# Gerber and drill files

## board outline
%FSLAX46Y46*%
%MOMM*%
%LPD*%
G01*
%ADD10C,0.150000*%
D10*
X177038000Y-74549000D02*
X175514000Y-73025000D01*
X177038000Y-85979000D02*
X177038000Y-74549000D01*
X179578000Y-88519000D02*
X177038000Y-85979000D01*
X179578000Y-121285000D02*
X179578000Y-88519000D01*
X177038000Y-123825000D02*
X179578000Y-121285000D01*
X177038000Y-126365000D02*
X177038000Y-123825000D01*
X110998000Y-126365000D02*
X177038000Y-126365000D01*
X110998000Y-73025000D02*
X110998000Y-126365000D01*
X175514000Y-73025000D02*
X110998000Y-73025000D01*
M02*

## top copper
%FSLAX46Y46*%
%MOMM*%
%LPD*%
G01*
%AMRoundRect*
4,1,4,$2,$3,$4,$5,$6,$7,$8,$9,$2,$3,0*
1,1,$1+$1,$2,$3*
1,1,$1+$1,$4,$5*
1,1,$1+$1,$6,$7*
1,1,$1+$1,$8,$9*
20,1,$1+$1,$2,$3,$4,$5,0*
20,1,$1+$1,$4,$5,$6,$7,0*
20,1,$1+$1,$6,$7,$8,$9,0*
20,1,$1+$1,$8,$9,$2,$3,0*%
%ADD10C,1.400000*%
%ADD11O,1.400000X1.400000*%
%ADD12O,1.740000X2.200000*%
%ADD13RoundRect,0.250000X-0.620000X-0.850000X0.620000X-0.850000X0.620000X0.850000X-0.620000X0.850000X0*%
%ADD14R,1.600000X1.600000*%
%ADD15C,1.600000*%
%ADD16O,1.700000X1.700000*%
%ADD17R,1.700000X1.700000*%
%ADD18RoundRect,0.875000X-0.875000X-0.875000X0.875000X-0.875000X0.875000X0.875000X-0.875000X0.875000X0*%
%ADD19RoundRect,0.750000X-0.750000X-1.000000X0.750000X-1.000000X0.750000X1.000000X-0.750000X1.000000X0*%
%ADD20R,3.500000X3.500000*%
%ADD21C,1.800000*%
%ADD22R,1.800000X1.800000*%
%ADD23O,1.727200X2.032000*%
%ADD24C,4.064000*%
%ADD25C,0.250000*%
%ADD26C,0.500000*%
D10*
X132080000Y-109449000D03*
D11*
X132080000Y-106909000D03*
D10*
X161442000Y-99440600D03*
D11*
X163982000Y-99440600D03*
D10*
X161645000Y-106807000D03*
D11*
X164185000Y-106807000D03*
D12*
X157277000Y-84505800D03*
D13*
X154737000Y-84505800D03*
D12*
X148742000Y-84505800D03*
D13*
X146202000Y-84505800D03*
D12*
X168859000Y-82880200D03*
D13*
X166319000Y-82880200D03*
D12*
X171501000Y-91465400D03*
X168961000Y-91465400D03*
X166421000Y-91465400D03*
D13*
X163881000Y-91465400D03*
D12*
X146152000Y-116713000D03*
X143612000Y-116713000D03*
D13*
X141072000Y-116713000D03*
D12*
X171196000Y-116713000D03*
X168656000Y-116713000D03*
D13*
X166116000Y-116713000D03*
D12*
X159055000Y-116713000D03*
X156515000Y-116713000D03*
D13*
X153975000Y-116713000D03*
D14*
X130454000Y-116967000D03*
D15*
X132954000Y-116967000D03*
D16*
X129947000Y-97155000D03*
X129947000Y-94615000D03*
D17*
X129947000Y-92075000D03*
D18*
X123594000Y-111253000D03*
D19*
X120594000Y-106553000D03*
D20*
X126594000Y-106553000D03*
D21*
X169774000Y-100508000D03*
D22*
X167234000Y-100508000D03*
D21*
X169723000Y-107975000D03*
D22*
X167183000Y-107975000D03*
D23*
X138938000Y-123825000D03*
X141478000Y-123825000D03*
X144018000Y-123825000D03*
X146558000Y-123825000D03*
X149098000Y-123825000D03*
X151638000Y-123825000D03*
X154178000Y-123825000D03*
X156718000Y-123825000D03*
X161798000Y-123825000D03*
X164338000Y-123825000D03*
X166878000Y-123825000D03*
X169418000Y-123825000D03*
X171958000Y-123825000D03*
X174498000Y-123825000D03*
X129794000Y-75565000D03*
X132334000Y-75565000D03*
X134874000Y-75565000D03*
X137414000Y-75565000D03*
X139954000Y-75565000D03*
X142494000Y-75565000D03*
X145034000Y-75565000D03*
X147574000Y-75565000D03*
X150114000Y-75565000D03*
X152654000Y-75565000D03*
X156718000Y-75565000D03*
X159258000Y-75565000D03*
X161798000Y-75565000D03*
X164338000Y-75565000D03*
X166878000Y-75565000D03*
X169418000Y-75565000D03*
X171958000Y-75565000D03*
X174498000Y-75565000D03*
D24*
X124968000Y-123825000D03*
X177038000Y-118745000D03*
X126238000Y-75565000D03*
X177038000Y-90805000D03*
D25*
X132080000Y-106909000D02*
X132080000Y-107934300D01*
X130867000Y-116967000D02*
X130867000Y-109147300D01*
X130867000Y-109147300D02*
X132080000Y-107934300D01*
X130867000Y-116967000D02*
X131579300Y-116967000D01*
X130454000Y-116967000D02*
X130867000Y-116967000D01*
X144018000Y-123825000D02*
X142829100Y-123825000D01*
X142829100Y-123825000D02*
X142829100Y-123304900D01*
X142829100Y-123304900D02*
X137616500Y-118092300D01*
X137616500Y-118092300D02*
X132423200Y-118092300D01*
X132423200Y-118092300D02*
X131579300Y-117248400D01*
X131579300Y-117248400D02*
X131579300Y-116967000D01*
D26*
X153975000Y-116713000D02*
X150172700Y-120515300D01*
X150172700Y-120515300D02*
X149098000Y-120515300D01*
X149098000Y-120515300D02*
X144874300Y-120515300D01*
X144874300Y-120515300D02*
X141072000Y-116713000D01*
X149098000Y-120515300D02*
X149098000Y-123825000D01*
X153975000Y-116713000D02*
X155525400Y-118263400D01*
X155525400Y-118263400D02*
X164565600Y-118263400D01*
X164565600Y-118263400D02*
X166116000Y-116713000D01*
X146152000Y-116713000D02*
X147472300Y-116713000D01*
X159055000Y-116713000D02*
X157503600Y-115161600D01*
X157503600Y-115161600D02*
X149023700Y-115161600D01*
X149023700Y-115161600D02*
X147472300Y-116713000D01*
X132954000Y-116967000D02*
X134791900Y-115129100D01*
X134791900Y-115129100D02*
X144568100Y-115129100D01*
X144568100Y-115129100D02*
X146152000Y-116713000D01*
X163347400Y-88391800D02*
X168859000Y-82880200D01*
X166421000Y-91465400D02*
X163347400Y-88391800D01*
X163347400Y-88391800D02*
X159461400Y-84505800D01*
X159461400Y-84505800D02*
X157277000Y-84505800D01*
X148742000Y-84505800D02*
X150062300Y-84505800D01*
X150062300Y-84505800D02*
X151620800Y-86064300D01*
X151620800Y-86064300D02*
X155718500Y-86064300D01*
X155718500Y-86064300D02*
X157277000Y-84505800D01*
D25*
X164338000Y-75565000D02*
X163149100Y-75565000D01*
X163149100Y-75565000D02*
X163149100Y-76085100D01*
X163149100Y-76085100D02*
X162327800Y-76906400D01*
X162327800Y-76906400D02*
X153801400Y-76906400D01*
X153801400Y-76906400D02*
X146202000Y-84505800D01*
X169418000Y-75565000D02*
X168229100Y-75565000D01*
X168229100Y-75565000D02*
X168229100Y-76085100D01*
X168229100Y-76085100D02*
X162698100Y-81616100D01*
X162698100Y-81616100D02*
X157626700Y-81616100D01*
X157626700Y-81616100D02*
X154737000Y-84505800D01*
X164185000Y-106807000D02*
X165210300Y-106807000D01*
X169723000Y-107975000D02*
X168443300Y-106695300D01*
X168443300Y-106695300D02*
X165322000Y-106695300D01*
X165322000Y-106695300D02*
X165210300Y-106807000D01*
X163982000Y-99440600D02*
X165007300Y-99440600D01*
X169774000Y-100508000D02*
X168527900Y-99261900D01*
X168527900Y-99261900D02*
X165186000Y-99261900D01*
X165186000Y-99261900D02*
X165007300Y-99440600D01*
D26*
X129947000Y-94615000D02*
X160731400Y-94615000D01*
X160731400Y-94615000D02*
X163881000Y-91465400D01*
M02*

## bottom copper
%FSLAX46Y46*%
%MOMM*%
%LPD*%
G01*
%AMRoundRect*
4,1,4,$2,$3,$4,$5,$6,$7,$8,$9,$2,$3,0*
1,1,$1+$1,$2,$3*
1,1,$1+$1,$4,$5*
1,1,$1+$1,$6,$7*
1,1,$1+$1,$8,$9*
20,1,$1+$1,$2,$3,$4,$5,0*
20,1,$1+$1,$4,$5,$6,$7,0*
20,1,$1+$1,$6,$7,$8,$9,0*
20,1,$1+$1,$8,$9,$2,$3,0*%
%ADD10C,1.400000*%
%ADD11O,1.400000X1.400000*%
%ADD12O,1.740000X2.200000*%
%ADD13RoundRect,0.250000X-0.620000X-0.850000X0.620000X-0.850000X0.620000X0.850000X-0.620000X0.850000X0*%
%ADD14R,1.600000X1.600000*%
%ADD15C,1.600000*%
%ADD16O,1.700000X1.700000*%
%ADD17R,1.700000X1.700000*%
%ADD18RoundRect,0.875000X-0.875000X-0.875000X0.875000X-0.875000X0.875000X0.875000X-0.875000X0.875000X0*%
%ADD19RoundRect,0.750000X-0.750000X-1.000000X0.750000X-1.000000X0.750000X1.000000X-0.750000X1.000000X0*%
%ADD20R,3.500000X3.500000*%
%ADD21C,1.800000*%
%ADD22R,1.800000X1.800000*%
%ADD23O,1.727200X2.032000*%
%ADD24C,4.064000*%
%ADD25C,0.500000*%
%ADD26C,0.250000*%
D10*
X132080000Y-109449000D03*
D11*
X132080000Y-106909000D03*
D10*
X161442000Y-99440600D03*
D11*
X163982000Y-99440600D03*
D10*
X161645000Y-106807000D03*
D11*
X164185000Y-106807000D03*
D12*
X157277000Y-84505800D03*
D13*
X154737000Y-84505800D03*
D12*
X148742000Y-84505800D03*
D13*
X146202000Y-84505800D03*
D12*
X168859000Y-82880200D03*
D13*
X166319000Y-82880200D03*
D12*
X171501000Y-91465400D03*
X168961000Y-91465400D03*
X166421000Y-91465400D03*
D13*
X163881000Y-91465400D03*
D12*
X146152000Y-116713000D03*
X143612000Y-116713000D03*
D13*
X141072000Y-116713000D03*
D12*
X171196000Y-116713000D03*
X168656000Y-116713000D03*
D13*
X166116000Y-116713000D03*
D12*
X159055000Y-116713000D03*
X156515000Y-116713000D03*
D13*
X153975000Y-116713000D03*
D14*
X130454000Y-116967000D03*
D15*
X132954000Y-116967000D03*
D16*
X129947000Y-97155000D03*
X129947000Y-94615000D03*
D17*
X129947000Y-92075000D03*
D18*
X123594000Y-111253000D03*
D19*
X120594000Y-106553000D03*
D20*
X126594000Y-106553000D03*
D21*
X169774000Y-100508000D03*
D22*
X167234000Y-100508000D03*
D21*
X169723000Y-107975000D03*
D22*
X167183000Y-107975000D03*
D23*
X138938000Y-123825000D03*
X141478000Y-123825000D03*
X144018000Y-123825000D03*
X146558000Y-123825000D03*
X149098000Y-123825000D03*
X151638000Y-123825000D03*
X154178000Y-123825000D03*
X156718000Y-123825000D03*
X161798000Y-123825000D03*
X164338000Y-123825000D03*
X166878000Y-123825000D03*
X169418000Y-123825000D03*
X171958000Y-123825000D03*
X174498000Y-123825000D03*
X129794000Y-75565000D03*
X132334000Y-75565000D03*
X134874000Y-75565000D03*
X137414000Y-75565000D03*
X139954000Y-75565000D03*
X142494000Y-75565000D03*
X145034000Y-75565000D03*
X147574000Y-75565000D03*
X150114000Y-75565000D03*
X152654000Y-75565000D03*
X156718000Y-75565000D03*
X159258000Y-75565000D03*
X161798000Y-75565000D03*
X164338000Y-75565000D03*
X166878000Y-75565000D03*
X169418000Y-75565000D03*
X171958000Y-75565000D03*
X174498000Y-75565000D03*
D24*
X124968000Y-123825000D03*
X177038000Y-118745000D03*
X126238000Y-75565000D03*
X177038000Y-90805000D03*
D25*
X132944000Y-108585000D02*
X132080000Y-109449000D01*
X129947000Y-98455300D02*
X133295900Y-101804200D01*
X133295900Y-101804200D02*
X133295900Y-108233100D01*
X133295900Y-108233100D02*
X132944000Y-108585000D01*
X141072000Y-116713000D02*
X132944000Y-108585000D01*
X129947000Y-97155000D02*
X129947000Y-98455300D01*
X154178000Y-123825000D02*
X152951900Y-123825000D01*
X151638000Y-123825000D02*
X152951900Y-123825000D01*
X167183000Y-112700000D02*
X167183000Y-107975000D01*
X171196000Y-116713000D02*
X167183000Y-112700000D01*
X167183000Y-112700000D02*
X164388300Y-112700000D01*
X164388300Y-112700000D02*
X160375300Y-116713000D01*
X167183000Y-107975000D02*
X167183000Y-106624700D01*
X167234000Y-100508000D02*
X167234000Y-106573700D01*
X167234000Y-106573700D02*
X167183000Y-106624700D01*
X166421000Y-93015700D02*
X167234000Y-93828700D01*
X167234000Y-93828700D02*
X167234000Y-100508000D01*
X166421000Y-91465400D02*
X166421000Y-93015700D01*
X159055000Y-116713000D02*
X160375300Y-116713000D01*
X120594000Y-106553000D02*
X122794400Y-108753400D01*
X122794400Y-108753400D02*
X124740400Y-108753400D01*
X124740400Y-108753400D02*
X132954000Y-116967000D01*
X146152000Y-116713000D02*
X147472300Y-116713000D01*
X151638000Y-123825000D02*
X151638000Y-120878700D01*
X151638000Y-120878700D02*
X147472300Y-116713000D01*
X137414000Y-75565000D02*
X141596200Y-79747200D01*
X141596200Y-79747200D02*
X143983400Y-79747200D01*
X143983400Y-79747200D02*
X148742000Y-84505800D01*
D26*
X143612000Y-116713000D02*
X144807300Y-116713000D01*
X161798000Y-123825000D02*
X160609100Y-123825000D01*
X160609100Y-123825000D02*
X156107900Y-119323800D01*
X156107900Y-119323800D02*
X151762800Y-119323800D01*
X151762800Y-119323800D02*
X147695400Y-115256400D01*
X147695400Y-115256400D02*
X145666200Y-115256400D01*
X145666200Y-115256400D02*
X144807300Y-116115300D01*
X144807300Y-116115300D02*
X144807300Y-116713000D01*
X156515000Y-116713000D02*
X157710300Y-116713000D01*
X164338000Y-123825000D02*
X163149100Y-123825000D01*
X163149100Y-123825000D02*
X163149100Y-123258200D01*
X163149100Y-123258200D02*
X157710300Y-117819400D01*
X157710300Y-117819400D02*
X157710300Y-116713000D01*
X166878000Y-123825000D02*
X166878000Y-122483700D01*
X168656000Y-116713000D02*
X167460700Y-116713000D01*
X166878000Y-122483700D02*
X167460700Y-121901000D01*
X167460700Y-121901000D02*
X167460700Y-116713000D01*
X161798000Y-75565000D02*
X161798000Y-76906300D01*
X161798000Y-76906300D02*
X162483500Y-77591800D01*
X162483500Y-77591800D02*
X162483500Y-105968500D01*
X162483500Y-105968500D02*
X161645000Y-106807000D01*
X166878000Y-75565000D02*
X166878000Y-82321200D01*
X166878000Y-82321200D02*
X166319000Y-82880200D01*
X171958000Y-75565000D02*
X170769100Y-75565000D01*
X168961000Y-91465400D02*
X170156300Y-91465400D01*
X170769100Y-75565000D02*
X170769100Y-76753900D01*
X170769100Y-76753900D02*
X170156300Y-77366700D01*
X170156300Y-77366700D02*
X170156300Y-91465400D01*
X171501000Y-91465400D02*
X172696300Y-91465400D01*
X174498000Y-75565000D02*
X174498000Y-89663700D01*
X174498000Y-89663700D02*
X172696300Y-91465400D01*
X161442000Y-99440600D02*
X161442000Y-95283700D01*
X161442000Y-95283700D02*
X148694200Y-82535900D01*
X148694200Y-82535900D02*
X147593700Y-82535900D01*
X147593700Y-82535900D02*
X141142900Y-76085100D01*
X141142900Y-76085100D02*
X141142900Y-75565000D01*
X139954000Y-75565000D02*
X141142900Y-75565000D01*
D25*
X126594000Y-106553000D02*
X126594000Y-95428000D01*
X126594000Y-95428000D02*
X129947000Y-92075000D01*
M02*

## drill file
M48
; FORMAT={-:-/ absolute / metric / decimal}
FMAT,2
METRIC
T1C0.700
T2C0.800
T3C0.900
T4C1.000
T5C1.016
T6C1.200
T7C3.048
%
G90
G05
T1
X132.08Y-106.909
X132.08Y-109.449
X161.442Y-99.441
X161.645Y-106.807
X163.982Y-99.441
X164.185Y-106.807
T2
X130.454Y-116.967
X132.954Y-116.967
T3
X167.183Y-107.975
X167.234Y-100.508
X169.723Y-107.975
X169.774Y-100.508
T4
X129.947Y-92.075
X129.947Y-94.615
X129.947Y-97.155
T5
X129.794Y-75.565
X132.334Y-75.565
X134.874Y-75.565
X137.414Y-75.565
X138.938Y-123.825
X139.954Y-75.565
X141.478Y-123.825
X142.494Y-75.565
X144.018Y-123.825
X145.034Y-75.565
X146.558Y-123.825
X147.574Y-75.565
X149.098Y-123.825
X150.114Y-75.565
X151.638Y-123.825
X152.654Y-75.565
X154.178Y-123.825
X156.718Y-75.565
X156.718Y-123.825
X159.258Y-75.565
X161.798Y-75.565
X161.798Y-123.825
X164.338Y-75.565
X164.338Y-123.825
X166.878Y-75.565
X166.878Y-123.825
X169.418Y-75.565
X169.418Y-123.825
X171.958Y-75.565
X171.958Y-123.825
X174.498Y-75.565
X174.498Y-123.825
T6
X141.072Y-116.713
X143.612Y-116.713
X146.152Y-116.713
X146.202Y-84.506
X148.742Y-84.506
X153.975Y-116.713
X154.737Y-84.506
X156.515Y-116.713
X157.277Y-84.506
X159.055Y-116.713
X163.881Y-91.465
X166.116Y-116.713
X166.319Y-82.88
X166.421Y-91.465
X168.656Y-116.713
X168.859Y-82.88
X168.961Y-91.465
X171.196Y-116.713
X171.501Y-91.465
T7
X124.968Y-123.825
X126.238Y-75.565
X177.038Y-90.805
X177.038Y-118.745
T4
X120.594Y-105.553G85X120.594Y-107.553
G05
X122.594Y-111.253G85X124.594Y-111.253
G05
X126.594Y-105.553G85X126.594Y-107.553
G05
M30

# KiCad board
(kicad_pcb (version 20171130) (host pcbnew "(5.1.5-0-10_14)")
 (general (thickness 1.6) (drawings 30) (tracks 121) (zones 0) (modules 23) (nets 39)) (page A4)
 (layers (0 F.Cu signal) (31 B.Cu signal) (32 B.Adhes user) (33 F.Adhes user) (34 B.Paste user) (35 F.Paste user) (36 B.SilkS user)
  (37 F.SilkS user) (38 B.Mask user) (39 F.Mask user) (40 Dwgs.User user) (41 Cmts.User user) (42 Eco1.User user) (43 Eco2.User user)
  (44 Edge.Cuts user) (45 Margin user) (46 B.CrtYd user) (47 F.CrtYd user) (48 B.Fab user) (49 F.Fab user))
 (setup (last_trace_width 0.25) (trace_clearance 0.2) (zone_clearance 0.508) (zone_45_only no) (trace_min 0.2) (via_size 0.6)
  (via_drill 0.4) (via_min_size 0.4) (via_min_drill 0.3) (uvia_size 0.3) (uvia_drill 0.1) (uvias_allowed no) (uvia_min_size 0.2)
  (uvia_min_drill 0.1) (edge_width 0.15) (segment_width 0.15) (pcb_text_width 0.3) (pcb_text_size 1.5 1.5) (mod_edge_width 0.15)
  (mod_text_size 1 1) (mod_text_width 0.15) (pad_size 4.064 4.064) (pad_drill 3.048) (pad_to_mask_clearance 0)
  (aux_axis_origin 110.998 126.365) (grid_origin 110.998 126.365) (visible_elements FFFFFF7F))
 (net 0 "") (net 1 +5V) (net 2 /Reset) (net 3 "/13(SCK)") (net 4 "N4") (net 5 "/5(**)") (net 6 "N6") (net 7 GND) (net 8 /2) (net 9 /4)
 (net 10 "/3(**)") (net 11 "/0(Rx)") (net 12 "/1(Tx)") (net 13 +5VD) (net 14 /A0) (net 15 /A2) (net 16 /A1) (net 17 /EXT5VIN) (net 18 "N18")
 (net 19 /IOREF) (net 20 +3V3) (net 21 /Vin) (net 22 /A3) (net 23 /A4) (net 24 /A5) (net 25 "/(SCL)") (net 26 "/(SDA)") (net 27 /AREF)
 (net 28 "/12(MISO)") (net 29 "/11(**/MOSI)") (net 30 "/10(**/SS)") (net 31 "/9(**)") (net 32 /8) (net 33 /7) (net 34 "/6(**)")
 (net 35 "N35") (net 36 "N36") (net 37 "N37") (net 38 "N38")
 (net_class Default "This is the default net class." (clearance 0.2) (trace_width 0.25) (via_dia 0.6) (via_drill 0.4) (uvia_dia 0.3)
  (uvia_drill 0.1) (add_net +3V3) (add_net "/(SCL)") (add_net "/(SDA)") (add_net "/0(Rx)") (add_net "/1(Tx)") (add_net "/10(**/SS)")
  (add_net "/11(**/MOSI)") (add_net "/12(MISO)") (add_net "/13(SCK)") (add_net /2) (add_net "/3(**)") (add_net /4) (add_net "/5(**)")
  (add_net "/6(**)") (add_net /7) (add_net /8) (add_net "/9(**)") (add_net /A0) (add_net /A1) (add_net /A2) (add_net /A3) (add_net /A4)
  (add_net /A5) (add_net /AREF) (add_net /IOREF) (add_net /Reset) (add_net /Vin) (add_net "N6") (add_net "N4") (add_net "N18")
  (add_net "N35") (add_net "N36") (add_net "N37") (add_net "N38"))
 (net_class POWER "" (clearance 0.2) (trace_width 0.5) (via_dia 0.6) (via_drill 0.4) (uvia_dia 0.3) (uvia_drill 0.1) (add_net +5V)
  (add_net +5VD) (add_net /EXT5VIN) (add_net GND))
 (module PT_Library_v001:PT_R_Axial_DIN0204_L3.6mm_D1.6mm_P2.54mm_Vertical (layer F.Cu) (at 132.08 109.449 90)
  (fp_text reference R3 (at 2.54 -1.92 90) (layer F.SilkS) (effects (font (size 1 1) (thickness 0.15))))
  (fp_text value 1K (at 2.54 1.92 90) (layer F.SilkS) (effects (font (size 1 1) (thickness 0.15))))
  (pad 1 thru_hole circle (at 0 0 90) (size 1.4 1.4) (drill 0.7) (layers *.Cu *.Mask) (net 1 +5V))
  (pad 2 thru_hole oval (at 2.54 0 90) (size 1.4 1.4) (drill 0.7) (layers *.Cu *.Mask) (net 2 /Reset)))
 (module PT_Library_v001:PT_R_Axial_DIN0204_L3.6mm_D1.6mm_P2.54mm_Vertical (layer F.Cu) (at 161.442 99.4406)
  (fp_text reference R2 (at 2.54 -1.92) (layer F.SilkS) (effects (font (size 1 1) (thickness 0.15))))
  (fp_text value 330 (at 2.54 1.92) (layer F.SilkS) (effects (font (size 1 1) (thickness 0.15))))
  (pad 1 thru_hole circle (at 0 0) (size 1.4 1.4) (drill 0.7) (layers *.Cu *.Mask) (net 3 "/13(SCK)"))
  (pad 2 thru_hole oval (at 2.54 0) (size 1.4 1.4) (drill 0.7) (layers *.Cu *.Mask) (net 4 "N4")))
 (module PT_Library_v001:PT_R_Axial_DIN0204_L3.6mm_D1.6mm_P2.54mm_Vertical (layer F.Cu) (at 161.645 106.807)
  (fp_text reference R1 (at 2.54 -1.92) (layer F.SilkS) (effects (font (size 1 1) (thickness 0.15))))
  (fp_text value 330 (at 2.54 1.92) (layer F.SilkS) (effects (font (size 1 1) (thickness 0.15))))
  (pad 1 thru_hole circle (at 0 0) (size 1.4 1.4) (drill 0.7) (layers *.Cu *.Mask) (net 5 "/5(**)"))
  (pad 2 thru_hole oval (at 2.54 0) (size 1.4 1.4) (drill 0.7) (layers *.Cu *.Mask) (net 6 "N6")))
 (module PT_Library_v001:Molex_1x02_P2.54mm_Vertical (layer F.Cu) (at 154.737 84.5058)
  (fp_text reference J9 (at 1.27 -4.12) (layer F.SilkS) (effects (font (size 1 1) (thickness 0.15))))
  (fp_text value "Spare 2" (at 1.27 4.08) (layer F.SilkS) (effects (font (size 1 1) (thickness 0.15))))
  (pad 2 thru_hole oval (at 2.54 0) (size 1.74 2.2) (drill 1.2) (layers *.Cu *.Mask) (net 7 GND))
  (pad 1 thru_hole roundrect (at 0 0) (size 1.74 2.2) (drill 1.2) (layers *.Cu *.Mask) (roundrect_rratio 0.143678) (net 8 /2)))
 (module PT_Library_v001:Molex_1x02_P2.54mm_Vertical (layer F.Cu) (at 146.202 84.5058)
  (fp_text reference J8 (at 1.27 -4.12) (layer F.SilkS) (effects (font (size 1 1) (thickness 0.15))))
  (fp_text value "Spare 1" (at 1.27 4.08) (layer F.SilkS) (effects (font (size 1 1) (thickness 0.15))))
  (pad 2 thru_hole oval (at 2.54 0) (size 1.74 2.2) (drill 1.2) (layers *.Cu *.Mask) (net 7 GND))
  (pad 1 thru_hole roundrect (at 0 0) (size 1.74 2.2) (drill 1.2) (layers *.Cu *.Mask) (roundrect_rratio 0.143678) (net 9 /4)))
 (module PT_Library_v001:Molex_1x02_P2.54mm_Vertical (layer F.Cu) (at 166.319 82.8802)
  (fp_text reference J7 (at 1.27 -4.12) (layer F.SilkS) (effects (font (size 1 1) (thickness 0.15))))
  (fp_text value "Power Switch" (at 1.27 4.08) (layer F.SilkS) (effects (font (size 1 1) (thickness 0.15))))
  (pad 2 thru_hole oval (at 2.54 0) (size 1.74 2.2) (drill 1.2) (layers *.Cu *.Mask) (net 7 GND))
  (pad 1 thru_hole roundrect (at 0 0) (size 1.74 2.2) (drill 1.2) (layers *.Cu *.Mask) (roundrect_rratio 0.143678) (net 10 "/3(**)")))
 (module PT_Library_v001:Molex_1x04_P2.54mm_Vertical (layer F.Cu) (at 163.881 91.4654)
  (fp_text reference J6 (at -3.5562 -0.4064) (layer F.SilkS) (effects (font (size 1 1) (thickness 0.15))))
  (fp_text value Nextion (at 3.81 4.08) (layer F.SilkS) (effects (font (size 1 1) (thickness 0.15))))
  (pad 4 thru_hole oval (at 7.62 0) (size 1.74 2.2) (drill 1.2) (layers *.Cu *.Mask) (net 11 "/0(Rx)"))
  (pad 3 thru_hole oval (at 5.08 0) (size 1.74 2.2) (drill 1.2) (layers *.Cu *.Mask) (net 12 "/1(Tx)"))
  (pad 2 thru_hole oval (at 2.54 0) (size 1.74 2.2) (drill 1.2) (layers *.Cu *.Mask) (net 7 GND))
  (pad 1 thru_hole roundrect (at 0 0) (size 1.74 2.2) (drill 1.2) (layers *.Cu *.Mask) (roundrect_rratio 0.143678) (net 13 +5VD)))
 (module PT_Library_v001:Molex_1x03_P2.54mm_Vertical (layer F.Cu) (at 141.072 116.713)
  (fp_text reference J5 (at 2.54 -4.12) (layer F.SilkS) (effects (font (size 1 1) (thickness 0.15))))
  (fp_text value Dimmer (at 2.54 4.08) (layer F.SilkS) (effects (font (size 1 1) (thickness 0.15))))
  (pad 3 thru_hole oval (at 5.08 0) (size 1.74 2.2) (drill 1.2) (layers *.Cu *.Mask) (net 7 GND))
  (pad 2 thru_hole oval (at 2.54 0) (size 1.74 2.2) (drill 1.2) (layers *.Cu *.Mask) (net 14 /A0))
  (pad 1 thru_hole roundrect (at 0 0) (size 1.74 2.2) (drill 1.2) (layers *.Cu *.Mask) (roundrect_rratio 0.143678) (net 1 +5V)))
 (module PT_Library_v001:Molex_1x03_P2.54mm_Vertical (layer F.Cu) (at 166.116 116.713)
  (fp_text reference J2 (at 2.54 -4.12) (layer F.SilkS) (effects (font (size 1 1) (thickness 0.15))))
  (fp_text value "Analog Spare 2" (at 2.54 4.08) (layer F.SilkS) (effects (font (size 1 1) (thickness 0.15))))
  (pad 3 thru_hole oval (at 5.08 0) (size 1.74 2.2) (drill 1.2) (layers *.Cu *.Mask) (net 7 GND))
  (pad 2 thru_hole oval (at 2.54 0) (size 1.74 2.2) (drill 1.2) (layers *.Cu *.Mask) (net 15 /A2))
  (pad 1 thru_hole roundrect (at 0 0) (size 1.74 2.2) (drill 1.2) (layers *.Cu *.Mask) (roundrect_rratio 0.143678) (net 1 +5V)))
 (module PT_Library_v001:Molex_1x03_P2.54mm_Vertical (layer F.Cu) (at 153.975 116.713)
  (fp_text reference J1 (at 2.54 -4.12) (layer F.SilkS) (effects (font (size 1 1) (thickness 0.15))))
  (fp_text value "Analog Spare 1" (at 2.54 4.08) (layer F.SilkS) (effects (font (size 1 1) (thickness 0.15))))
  (pad 3 thru_hole oval (at 5.08 0) (size 1.74 2.2) (drill 1.2) (layers *.Cu *.Mask) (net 7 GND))
  (pad 2 thru_hole oval (at 2.54 0) (size 1.74 2.2) (drill 1.2) (layers *.Cu *.Mask) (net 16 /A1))
  (pad 1 thru_hole roundrect (at 0 0) (size 1.74 2.2) (drill 1.2) (layers *.Cu *.Mask) (roundrect_rratio 0.143678) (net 1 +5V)))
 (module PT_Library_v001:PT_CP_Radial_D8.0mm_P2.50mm (layer F.Cu) (at 130.454 116.967)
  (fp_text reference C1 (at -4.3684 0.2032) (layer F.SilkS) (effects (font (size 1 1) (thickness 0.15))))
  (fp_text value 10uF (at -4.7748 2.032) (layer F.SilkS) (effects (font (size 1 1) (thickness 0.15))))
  (pad 1 thru_hole rect (at 0 0) (size 1.6 1.6) (drill 0.8) (layers *.Cu *.Mask) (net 2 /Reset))
  (pad 2 thru_hole circle (at 2.5 0) (size 1.6 1.6) (drill 0.8) (layers *.Cu *.Mask) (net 7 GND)))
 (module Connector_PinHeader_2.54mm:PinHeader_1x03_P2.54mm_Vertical (layer F.Cu) (at 129.947 92.075)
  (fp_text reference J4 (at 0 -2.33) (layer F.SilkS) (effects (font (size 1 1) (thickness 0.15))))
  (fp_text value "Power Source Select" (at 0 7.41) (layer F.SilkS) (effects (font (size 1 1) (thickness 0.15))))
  (pad 3 thru_hole oval (at 0 5.08) (size 1.7 1.7) (drill 1) (layers *.Cu *.Mask) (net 1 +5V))
  (pad 2 thru_hole oval (at 0 2.54) (size 1.7 1.7) (drill 1) (layers *.Cu *.Mask) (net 13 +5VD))
  (pad 1 thru_hole rect (at 0 0) (size 1.7 1.7) (drill 1) (layers *.Cu *.Mask) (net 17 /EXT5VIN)))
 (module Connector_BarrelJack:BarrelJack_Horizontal (layer F.Cu) (at 126.594 106.553)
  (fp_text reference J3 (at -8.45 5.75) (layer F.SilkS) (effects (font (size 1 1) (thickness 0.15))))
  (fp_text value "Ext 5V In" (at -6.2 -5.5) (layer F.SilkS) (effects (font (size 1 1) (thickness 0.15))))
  (pad 3 thru_hole roundrect (at -3 4.7) (size 3.5 3.5) (drill oval 3 1) (layers *.Cu *.Mask) (roundrect_rratio 0.25))
  (pad 2 thru_hole roundrect (at -6 0) (size 3 3.5) (drill oval 1 3) (layers *.Cu *.Mask) (roundrect_rratio 0.25) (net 7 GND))
  (pad 1 thru_hole rect (at 0 0) (size 3.5 3.5) (drill oval 1 3) (layers *.Cu *.Mask) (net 17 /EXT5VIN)))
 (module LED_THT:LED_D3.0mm (layer F.Cu) (at 167.234 100.508)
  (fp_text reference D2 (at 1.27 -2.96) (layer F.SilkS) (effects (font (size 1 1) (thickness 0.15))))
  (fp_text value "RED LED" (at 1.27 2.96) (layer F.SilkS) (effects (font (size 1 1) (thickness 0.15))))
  (pad 2 thru_hole circle (at 2.54 0) (size 1.8 1.8) (drill 0.9) (layers *.Cu *.Mask) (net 4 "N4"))
  (pad 1 thru_hole rect (at 0 0) (size 1.8 1.8) (drill 0.9) (layers *.Cu *.Mask) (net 7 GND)))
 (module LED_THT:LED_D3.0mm (layer F.Cu) (at 167.183 107.975)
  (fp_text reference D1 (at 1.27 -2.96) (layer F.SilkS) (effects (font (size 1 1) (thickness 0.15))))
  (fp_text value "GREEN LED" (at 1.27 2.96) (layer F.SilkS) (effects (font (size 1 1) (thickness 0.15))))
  (pad 2 thru_hole circle (at 2.54 0) (size 1.8 1.8) (drill 0.9) (layers *.Cu *.Mask) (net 6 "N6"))
  (pad 1 thru_hole rect (at 0 0) (size 1.8 1.8) (drill 0.9) (layers *.Cu *.Mask) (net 7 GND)))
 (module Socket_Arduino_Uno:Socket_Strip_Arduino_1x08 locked (layer F.Cu) (at 138.938 123.825)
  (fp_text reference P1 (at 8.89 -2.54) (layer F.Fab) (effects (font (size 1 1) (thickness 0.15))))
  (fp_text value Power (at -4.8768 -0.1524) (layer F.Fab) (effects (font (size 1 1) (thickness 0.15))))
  (pad 1 thru_hole oval (at 0 0) (size 1.7272 2.032) (drill 1.016) (layers *.Cu *.Mask F.SilkS) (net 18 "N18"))
  (pad 2 thru_hole oval (at 2.54 0) (size 1.7272 2.032) (drill 1.016) (layers *.Cu *.Mask F.SilkS) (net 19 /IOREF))
  (pad 3 thru_hole oval (at 5.08 0) (size 1.7272 2.032) (drill 1.016) (layers *.Cu *.Mask F.SilkS) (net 2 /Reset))
  (pad 4 thru_hole oval (at 7.62 0) (size 1.7272 2.032) (drill 1.016) (layers *.Cu *.Mask F.SilkS) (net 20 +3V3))
  (pad 5 thru_hole oval (at 10.16 0) (size 1.7272 2.032) (drill 1.016) (layers *.Cu *.Mask F.SilkS) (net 1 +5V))
  (pad 6 thru_hole oval (at 12.7 0) (size 1.7272 2.032) (drill 1.016) (layers *.Cu *.Mask F.SilkS) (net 7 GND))
  (pad 7 thru_hole oval (at 15.24 0) (size 1.7272 2.032) (drill 1.016) (layers *.Cu *.Mask F.SilkS) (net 7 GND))
  (pad 8 thru_hole oval (at 17.78 0) (size 1.7272 2.032) (drill 1.016) (layers *.Cu *.Mask F.SilkS) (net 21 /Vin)))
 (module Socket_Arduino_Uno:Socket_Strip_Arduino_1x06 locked (layer F.Cu) (at 161.798 123.825)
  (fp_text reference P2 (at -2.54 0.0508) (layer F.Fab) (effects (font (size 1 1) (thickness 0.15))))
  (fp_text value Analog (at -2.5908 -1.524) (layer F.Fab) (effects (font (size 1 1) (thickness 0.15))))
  (pad 1 thru_hole oval (at 0 0) (size 1.7272 2.032) (drill 1.016) (layers *.Cu *.Mask F.SilkS) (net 14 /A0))
  (pad 2 thru_hole oval (at 2.54 0) (size 1.7272 2.032) (drill 1.016) (layers *.Cu *.Mask F.SilkS) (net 16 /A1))
  (pad 3 thru_hole oval (at 5.08 0) (size 1.7272 2.032) (drill 1.016) (layers *.Cu *.Mask F.SilkS) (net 15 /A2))
  (pad 4 thru_hole oval (at 7.62 0) (size 1.7272 2.032) (drill 1.016) (layers *.Cu *.Mask F.SilkS) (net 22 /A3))
  (pad 5 thru_hole oval (at 10.16 0) (size 1.7272 2.032) (drill 1.016) (layers *.Cu *.Mask F.SilkS) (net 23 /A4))
  (pad 6 thru_hole oval (at 12.7 0) (size 1.7272 2.032) (drill 1.016) (layers *.Cu *.Mask F.SilkS) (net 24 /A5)))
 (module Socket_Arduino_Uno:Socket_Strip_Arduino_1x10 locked (layer F.Cu) (at 129.794 75.565)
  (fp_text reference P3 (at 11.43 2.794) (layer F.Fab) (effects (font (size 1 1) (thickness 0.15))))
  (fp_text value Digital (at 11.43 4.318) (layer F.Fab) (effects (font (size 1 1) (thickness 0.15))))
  (pad 1 thru_hole oval (at 0 0) (size 1.7272 2.032) (drill 1.016) (layers *.Cu *.Mask F.SilkS) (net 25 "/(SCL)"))
  (pad 2 thru_hole oval (at 2.54 0) (size 1.7272 2.032) (drill 1.016) (layers *.Cu *.Mask F.SilkS) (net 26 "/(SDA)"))
  (pad 3 thru_hole oval (at 5.08 0) (size 1.7272 2.032) (drill 1.016) (layers *.Cu *.Mask F.SilkS) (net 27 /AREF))
  (pad 4 thru_hole oval (at 7.62 0) (size 1.7272 2.032) (drill 1.016) (layers *.Cu *.Mask F.SilkS) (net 7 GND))
  (pad 5 thru_hole oval (at 10.16 0) (size 1.7272 2.032) (drill 1.016) (layers *.Cu *.Mask F.SilkS) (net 3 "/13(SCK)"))
  (pad 6 thru_hole oval (at 12.7 0) (size 1.7272 2.032) (drill 1.016) (layers *.Cu *.Mask F.SilkS) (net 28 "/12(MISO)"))
  (pad 7 thru_hole oval (at 15.24 0) (size 1.7272 2.032) (drill 1.016) (layers *.Cu *.Mask F.SilkS) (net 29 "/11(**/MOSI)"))
  (pad 8 thru_hole oval (at 17.78 0) (size 1.7272 2.032) (drill 1.016) (layers *.Cu *.Mask F.SilkS) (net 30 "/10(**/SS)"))
  (pad 9 thru_hole oval (at 20.32 0) (size 1.7272 2.032) (drill 1.016) (layers *.Cu *.Mask F.SilkS) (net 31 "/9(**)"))
  (pad 10 thru_hole oval (at 22.86 0) (size 1.7272 2.032) (drill 1.016) (layers *.Cu *.Mask F.SilkS) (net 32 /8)))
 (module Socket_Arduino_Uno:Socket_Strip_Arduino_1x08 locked (layer F.Cu) (at 156.718 75.565)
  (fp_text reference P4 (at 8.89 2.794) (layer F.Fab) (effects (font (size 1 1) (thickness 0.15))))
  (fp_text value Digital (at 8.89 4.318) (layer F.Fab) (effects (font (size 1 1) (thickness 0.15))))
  (pad 1 thru_hole oval (at 0 0) (size 1.7272 2.032) (drill 1.016) (layers *.Cu *.Mask F.SilkS) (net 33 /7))
  (pad 2 thru_hole oval (at 2.54 0) (size 1.7272 2.032) (drill 1.016) (layers *.Cu *.Mask F.SilkS) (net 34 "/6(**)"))
  (pad 3 thru_hole oval (at 5.08 0) (size 1.7272 2.032) (drill 1.016) (layers *.Cu *.Mask F.SilkS) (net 5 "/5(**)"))
  (pad 4 thru_hole oval (at 7.62 0) (size 1.7272 2.032) (drill 1.016) (layers *.Cu *.Mask F.SilkS) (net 9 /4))
  (pad 5 thru_hole oval (at 10.16 0) (size 1.7272 2.032) (drill 1.016) (layers *.Cu *.Mask F.SilkS) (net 10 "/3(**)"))
  (pad 6 thru_hole oval (at 12.7 0) (size 1.7272 2.032) (drill 1.016) (layers *.Cu *.Mask F.SilkS) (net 8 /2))
  (pad 7 thru_hole oval (at 15.24 0) (size 1.7272 2.032) (drill 1.016) (layers *.Cu *.Mask F.SilkS) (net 12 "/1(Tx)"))
  (pad 8 thru_hole oval (at 17.78 0) (size 1.7272 2.032) (drill 1.016) (layers *.Cu *.Mask F.SilkS) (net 11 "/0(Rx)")))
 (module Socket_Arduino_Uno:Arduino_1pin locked (layer F.Cu) (at 124.968 123.825)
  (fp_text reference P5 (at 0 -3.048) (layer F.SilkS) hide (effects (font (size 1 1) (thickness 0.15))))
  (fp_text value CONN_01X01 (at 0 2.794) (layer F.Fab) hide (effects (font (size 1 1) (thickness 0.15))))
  (pad 1 thru_hole circle (at 0 0) (size 4.064 4.064) (drill 3.048) (layers *.Cu *.Mask F.SilkS) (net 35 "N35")))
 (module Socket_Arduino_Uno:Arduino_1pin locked (layer F.Cu) (at 177.038 118.745)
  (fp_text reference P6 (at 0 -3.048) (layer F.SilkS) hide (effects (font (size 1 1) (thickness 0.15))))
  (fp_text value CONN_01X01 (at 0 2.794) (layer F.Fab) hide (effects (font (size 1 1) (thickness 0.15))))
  (pad 1 thru_hole circle (at 0 0) (size 4.064 4.064) (drill 3.048) (layers *.Cu *.Mask F.SilkS) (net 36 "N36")))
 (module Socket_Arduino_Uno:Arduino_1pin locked (layer F.Cu) (at 126.238 75.565)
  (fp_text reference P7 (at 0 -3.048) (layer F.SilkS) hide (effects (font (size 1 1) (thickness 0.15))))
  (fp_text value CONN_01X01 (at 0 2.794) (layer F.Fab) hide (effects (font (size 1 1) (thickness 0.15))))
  (pad 1 thru_hole circle (at 0 0) (size 4.064 4.064) (drill 3.048) (layers *.Cu *.Mask F.SilkS) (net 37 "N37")))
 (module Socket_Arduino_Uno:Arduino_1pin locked (layer F.Cu) (at 177.038 90.805)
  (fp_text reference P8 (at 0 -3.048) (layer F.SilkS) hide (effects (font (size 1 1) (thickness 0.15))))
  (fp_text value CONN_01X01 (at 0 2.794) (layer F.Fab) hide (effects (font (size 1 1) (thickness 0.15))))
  (pad 1 thru_hole circle (at 0 0) (size 4.064 4.064) (drill 3.048) (layers *.Cu *.Mask F.SilkS) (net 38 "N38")))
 (gr_line (start 177.038 74.549) (end 175.514 73.025) (angle 90) (layer Edge.Cuts) (width 0.15))
 (gr_line (start 177.038 85.979) (end 177.038 74.549) (angle 90) (layer Edge.Cuts) (width 0.15))
 (gr_line (start 179.578 88.519) (end 177.038 85.979) (angle 90) (layer Edge.Cuts) (width 0.15))
 (gr_line (start 179.578 121.285) (end 179.578 88.519) (angle 90) (layer Edge.Cuts) (width 0.15))
 (gr_line (start 177.038 123.825) (end 179.578 121.285) (angle 90) (layer Edge.Cuts) (width 0.15))
 (gr_line (start 177.038 126.365) (end 177.038 123.825) (angle 90) (layer Edge.Cuts) (width 0.15))
 (gr_line (start 110.998 126.365) (end 177.038 126.365) (angle 90) (layer Edge.Cuts) (width 0.15))
 (gr_line (start 110.998 73.025) (end 110.998 126.365) (angle 90) (layer Edge.Cuts) (width 0.15))
 (gr_line (start 175.514 73.025) (end 110.998 73.025) (angle 90) (layer Edge.Cuts) (width 0.15))
 (segment (start 132.08 106.909) (end 132.08 107.9343) (width 0.25) (layer F.Cu) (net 2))
 (segment (start 130.867 116.967) (end 130.867 109.1473) (width 0.25) (layer F.Cu) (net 2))
 (segment (start 130.867 109.1473) (end 132.08 107.9343) (width 0.25) (layer F.Cu) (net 2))
 (segment (start 130.867 116.967) (end 131.5793 116.967) (width 0.25) (layer F.Cu) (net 2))
 (segment (start 130.454 116.967) (end 130.867 116.967) (width 0.25) (layer F.Cu) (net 2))
 (segment (start 144.018 123.825) (end 142.8291 123.825) (width 0.25) (layer F.Cu) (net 2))
 (segment (start 142.8291 123.825) (end 142.8291 123.3049) (width 0.25) (layer F.Cu) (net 2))
 (segment (start 142.8291 123.3049) (end 137.6165 118.0923) (width 0.25) (layer F.Cu) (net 2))
 (segment (start 137.6165 118.0923) (end 132.4232 118.0923) (width 0.25) (layer F.Cu) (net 2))
 (segment (start 132.4232 118.0923) (end 131.5793 117.2484) (width 0.25) (layer F.Cu) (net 2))
 (segment (start 131.5793 117.2484) (end 131.5793 116.967) (width 0.25) (layer F.Cu) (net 2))
 (segment (start 153.975 116.713) (end 150.1727 120.5153) (width 0.5) (layer F.Cu) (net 1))
 (segment (start 150.1727 120.5153) (end 149.098 120.5153) (width 0.5) (layer F.Cu) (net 1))
 (segment (start 149.098 120.5153) (end 144.8743 120.5153) (width 0.5) (layer F.Cu) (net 1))
 (segment (start 144.8743 120.5153) (end 141.072 116.713) (width 0.5) (layer F.Cu) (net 1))
 (segment (start 149.098 120.5153) (end 149.098 123.825) (width 0.5) (layer F.Cu) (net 1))
 (segment (start 153.975 116.713) (end 155.5254 118.2634) (width 0.5) (layer F.Cu) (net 1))
 (segment (start 155.5254 118.2634) (end 164.5656 118.2634) (width 0.5) (layer F.Cu) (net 1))
 (segment (start 164.5656 118.2634) (end 166.116 116.713) (width 0.5) (layer F.Cu) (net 1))
 (segment (start 132.944 108.585) (end 132.08 109.449) (width 0.5) (layer B.Cu) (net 1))
 (segment (start 129.947 98.4553) (end 133.2959 101.8042) (width 0.5) (layer B.Cu) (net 1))
 (segment (start 133.2959 101.8042) (end 133.2959 108.2331) (width 0.5) (layer B.Cu) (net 1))
 (segment (start 133.2959 108.2331) (end 132.944 108.585) (width 0.5) (layer B.Cu) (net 1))
 (segment (start 141.072 116.713) (end 132.944 108.585) (width 0.5) (layer B.Cu) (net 1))
 (segment (start 129.947 97.155) (end 129.947 98.4553) (width 0.5) (layer B.Cu) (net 1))
 (segment (start 146.152 116.713) (end 147.4723 116.713) (width 0.5) (layer F.Cu) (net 7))
 (segment (start 159.055 116.713) (end 157.5036 115.1616) (width 0.5) (layer F.Cu) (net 7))
 (segment (start 157.5036 115.1616) (end 149.0237 115.1616) (width 0.5) (layer F.Cu) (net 7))
 (segment (start 149.0237 115.1616) (end 147.4723 116.713) (width 0.5) (layer F.Cu) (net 7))
 (segment (start 132.954 116.967) (end 134.7919 115.1291) (width 0.5) (layer F.Cu) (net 7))
 (segment (start 134.7919 115.1291) (end 144.5681 115.1291) (width 0.5) (layer F.Cu) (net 7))
 (segment (start 144.5681 115.1291) (end 146.152 116.713) (width 0.5) (layer F.Cu) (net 7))
 (segment (start 163.3474 88.3918) (end 168.859 82.8802) (width 0.5) (layer F.Cu) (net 7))
 (segment (start 166.421 91.4654) (end 163.3474 88.3918) (width 0.5) (layer F.Cu) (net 7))
 (segment (start 163.3474 88.3918) (end 159.4614 84.5058) (width 0.5) (layer F.Cu) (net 7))
 (segment (start 159.4614 84.5058) (end 157.277 84.5058) (width 0.5) (layer F.Cu) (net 7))
 (segment (start 148.742 84.5058) (end 150.0623 84.5058) (width 0.5) (layer F.Cu) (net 7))
 (segment (start 150.0623 84.5058) (end 151.6208 86.0643) (width 0.5) (layer F.Cu) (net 7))
 (segment (start 151.6208 86.0643) (end 155.7185 86.0643) (width 0.5) (layer F.Cu) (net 7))
 (segment (start 155.7185 86.0643) (end 157.277 84.5058) (width 0.5) (layer F.Cu) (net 7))
 (segment (start 154.178 123.825) (end 152.9519 123.825) (width 0.5) (layer B.Cu) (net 7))
 (segment (start 151.638 123.825) (end 152.9519 123.825) (width 0.5) (layer B.Cu) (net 7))
 (segment (start 167.183 112.7) (end 167.183 107.975) (width 0.5) (layer B.Cu) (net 7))
 (segment (start 171.196 116.713) (end 167.183 112.7) (width 0.5) (layer B.Cu) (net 7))
 (segment (start 167.183 112.7) (end 164.3883 112.7) (width 0.5) (layer B.Cu) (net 7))
 (segment (start 164.3883 112.7) (end 160.3753 116.713) (width 0.5) (layer B.Cu) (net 7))
 (segment (start 167.183 107.975) (end 167.183 106.6247) (width 0.5) (layer B.Cu) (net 7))
 (segment (start 167.234 100.508) (end 167.234 106.5737) (width 0.5) (layer B.Cu) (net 7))
 (segment (start 167.234 106.5737) (end 167.183 106.6247) (width 0.5) (layer B.Cu) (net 7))
 (segment (start 166.421 93.0157) (end 167.234 93.8287) (width 0.5) (layer B.Cu) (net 7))
 (segment (start 167.234 93.8287) (end 167.234 100.508) (width 0.5) (layer B.Cu) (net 7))
 (segment (start 166.421 91.4654) (end 166.421 93.0157) (width 0.5) (layer B.Cu) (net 7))
 (segment (start 159.055 116.713) (end 160.3753 116.713) (width 0.5) (layer B.Cu) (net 7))
 (segment (start 120.594 106.553) (end 122.7944 108.7534) (width 0.5) (layer B.Cu) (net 7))
 (segment (start 122.7944 108.7534) (end 124.7404 108.7534) (width 0.5) (layer B.Cu) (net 7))
 (segment (start 124.7404 108.7534) (end 132.954 116.967) (width 0.5) (layer B.Cu) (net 7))
 (segment (start 146.152 116.713) (end 147.4723 116.713) (width 0.5) (layer B.Cu) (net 7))
 (segment (start 151.638 123.825) (end 151.638 120.8787) (width 0.5) (layer B.Cu) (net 7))
 (segment (start 151.638 120.8787) (end 147.4723 116.713) (width 0.5) (layer B.Cu) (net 7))
 (segment (start 137.414 75.565) (end 141.5962 79.7472) (width 0.5) (layer B.Cu) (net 7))
 (segment (start 141.5962 79.7472) (end 143.9834 79.7472) (width 0.5) (layer B.Cu) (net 7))
 (segment (start 143.9834 79.7472) (end 148.742 84.5058) (width 0.5) (layer B.Cu) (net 7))
 (segment (start 143.612 116.713) (end 144.8073 116.713) (width 0.25) (layer B.Cu) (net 14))
 (segment (start 161.798 123.825) (end 160.6091 123.825) (width 0.25) (layer B.Cu) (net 14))
 (segment (start 160.6091 123.825) (end 156.1079 119.3238) (width 0.25) (layer B.Cu) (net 14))
 (segment (start 156.1079 119.3238) (end 151.7628 119.3238) (width 0.25) (layer B.Cu) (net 14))
 (segment (start 151.7628 119.3238) (end 147.6954 115.2564) (width 0.25) (layer B.Cu) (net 14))
 (segment (start 147.6954 115.2564) (end 145.6662 115.2564) (width 0.25) (layer B.Cu) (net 14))
 (segment (start 145.6662 115.2564) (end 144.8073 116.1153) (width 0.25) (layer B.Cu) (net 14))
 (segment (start 144.8073 116.1153) (end 144.8073 116.713) (width 0.25) (layer B.Cu) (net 14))
 (segment (start 156.515 116.713) (end 157.7103 116.713) (width 0.25) (layer B.Cu) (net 16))
 (segment (start 164.338 123.825) (end 163.1491 123.825) (width 0.25) (layer B.Cu) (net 16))
 (segment (start 163.1491 123.825) (end 163.1491 123.2582) (width 0.25) (layer B.Cu) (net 16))
 (segment (start 163.1491 123.2582) (end 157.7103 117.8194) (width 0.25) (layer B.Cu) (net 16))
 (segment (start 157.7103 117.8194) (end 157.7103 116.713) (width 0.25) (layer B.Cu) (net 16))
 (segment (start 166.878 123.825) (end 166.878 122.4837) (width 0.25) (layer B.Cu) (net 15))
 (segment (start 168.656 116.713) (end 167.4607 116.713) (width 0.25) (layer B.Cu) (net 15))
 (segment (start 166.878 122.4837) (end 167.4607 121.901) (width 0.25) (layer B.Cu) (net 15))
 (segment (start 167.4607 121.901) (end 167.4607 116.713) (width 0.25) (layer B.Cu) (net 15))
 (segment (start 161.798 75.565) (end 161.798 76.9063) (width 0.25) (layer B.Cu) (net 5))
 (segment (start 161.798 76.9063) (end 162.4835 77.5918) (width 0.25) (layer B.Cu) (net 5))
 (segment (start 162.4835 77.5918) (end 162.4835 105.9685) (width 0.25) (layer B.Cu) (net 5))
 (segment (start 162.4835 105.9685) (end 161.645 106.807) (width 0.25) (layer B.Cu) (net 5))
 (segment (start 164.338 75.565) (end 163.1491 75.565) (width 0.25) (layer F.Cu) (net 9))
 (segment (start 163.1491 75.565) (end 163.1491 76.0851) (width 0.25) (layer F.Cu) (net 9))
 (segment (start 163.1491 76.0851) (end 162.3278 76.9064) (width 0.25) (layer F.Cu) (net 9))
 (segment (start 162.3278 76.9064) (end 153.8014 76.9064) (width 0.25) (layer F.Cu) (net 9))
 (segment (start 153.8014 76.9064) (end 146.202 84.5058) (width 0.25) (layer F.Cu) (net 9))
 (segment (start 166.878 75.565) (end 166.878 82.3212) (width 0.25) (layer B.Cu) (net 10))
 (segment (start 166.878 82.3212) (end 166.319 82.8802) (width 0.25) (layer B.Cu) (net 10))
 (segment (start 169.418 75.565) (end 168.2291 75.565) (width 0.25) (layer F.Cu) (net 8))
 (segment (start 168.2291 75.565) (end 168.2291 76.0851) (width 0.25) (layer F.Cu) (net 8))
 (segment (start 168.2291 76.0851) (end 162.6981 81.6161) (width 0.25) (layer F.Cu) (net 8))
 (segment (start 162.6981 81.6161) (end 157.6267 81.6161) (width 0.25) (layer F.Cu) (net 8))
 (segment (start 157.6267 81.6161) (end 154.737 84.5058) (width 0.25) (layer F.Cu) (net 8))
 (segment (start 171.958 75.565) (end 170.7691 75.565) (width 0.25) (layer B.Cu) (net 12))
 (segment (start 168.961 91.4654) (end 170.1563 91.4654) (width 0.25) (layer B.Cu) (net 12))
 (segment (start 170.7691 75.565) (end 170.7691 76.7539) (width 0.25) (layer B.Cu) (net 12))
 (segment (start 170.7691 76.7539) (end 170.1563 77.3667) (width 0.25) (layer B.Cu) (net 12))
 (segment (start 170.1563 77.3667) (end 170.1563 91.4654) (width 0.25) (layer B.Cu) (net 12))
 (segment (start 171.501 91.4654) (end 172.6963 91.4654) (width 0.25) (layer B.Cu) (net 11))
 (segment (start 174.498 75.565) (end 174.498 89.6637) (width 0.25) (layer B.Cu) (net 11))
 (segment (start 174.498 89.6637) (end 172.6963 91.4654) (width 0.25) (layer B.Cu) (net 11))
 (segment (start 161.442 99.4406) (end 161.442 95.2837) (width 0.25) (layer B.Cu) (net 3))
 (segment (start 161.442 95.2837) (end 148.6942 82.5359) (width 0.25) (layer B.Cu) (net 3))
 (segment (start 148.6942 82.5359) (end 147.5937 82.5359) (width 0.25) (layer B.Cu) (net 3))
 (segment (start 147.5937 82.5359) (end 141.1429 76.0851) (width 0.25) (layer B.Cu) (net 3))
 (segment (start 141.1429 76.0851) (end 141.1429 75.565) (width 0.25) (layer B.Cu) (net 3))
 (segment (start 139.954 75.565) (end 141.1429 75.565) (width 0.25) (layer B.Cu) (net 3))
 (segment (start 164.185 106.807) (end 165.2103 106.807) (width 0.25) (layer F.Cu) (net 6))
 (segment (start 169.723 107.975) (end 168.4433 106.6953) (width 0.25) (layer F.Cu) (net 6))
 (segment (start 168.4433 106.6953) (end 165.322 106.6953) (width 0.25) (layer F.Cu) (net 6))
 (segment (start 165.322 106.6953) (end 165.2103 106.807) (width 0.25) (layer F.Cu) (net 6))
 (segment (start 163.982 99.4406) (end 165.0073 99.4406) (width 0.25) (layer F.Cu) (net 4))
 (segment (start 169.774 100.508) (end 168.5279 99.2619) (width 0.25) (layer F.Cu) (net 4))
 (segment (start 168.5279 99.2619) (end 165.186 99.2619) (width 0.25) (layer F.Cu) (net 4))
 (segment (start 165.186 99.2619) (end 165.0073 99.4406) (width 0.25) (layer F.Cu) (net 4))
 (segment (start 129.947 94.615) (end 160.7314 94.615) (width 0.5) (layer F.Cu) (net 13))
 (segment (start 160.7314 94.615) (end 163.881 91.4654) (width 0.5) (layer F.Cu) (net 13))
 (segment (start 126.594 106.553) (end 126.594 95.428) (width 0.5) (layer B.Cu) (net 17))
 (segment (start 126.594 95.428) (end 129.947 92.075) (width 0.5) (layer B.Cu) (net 17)))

